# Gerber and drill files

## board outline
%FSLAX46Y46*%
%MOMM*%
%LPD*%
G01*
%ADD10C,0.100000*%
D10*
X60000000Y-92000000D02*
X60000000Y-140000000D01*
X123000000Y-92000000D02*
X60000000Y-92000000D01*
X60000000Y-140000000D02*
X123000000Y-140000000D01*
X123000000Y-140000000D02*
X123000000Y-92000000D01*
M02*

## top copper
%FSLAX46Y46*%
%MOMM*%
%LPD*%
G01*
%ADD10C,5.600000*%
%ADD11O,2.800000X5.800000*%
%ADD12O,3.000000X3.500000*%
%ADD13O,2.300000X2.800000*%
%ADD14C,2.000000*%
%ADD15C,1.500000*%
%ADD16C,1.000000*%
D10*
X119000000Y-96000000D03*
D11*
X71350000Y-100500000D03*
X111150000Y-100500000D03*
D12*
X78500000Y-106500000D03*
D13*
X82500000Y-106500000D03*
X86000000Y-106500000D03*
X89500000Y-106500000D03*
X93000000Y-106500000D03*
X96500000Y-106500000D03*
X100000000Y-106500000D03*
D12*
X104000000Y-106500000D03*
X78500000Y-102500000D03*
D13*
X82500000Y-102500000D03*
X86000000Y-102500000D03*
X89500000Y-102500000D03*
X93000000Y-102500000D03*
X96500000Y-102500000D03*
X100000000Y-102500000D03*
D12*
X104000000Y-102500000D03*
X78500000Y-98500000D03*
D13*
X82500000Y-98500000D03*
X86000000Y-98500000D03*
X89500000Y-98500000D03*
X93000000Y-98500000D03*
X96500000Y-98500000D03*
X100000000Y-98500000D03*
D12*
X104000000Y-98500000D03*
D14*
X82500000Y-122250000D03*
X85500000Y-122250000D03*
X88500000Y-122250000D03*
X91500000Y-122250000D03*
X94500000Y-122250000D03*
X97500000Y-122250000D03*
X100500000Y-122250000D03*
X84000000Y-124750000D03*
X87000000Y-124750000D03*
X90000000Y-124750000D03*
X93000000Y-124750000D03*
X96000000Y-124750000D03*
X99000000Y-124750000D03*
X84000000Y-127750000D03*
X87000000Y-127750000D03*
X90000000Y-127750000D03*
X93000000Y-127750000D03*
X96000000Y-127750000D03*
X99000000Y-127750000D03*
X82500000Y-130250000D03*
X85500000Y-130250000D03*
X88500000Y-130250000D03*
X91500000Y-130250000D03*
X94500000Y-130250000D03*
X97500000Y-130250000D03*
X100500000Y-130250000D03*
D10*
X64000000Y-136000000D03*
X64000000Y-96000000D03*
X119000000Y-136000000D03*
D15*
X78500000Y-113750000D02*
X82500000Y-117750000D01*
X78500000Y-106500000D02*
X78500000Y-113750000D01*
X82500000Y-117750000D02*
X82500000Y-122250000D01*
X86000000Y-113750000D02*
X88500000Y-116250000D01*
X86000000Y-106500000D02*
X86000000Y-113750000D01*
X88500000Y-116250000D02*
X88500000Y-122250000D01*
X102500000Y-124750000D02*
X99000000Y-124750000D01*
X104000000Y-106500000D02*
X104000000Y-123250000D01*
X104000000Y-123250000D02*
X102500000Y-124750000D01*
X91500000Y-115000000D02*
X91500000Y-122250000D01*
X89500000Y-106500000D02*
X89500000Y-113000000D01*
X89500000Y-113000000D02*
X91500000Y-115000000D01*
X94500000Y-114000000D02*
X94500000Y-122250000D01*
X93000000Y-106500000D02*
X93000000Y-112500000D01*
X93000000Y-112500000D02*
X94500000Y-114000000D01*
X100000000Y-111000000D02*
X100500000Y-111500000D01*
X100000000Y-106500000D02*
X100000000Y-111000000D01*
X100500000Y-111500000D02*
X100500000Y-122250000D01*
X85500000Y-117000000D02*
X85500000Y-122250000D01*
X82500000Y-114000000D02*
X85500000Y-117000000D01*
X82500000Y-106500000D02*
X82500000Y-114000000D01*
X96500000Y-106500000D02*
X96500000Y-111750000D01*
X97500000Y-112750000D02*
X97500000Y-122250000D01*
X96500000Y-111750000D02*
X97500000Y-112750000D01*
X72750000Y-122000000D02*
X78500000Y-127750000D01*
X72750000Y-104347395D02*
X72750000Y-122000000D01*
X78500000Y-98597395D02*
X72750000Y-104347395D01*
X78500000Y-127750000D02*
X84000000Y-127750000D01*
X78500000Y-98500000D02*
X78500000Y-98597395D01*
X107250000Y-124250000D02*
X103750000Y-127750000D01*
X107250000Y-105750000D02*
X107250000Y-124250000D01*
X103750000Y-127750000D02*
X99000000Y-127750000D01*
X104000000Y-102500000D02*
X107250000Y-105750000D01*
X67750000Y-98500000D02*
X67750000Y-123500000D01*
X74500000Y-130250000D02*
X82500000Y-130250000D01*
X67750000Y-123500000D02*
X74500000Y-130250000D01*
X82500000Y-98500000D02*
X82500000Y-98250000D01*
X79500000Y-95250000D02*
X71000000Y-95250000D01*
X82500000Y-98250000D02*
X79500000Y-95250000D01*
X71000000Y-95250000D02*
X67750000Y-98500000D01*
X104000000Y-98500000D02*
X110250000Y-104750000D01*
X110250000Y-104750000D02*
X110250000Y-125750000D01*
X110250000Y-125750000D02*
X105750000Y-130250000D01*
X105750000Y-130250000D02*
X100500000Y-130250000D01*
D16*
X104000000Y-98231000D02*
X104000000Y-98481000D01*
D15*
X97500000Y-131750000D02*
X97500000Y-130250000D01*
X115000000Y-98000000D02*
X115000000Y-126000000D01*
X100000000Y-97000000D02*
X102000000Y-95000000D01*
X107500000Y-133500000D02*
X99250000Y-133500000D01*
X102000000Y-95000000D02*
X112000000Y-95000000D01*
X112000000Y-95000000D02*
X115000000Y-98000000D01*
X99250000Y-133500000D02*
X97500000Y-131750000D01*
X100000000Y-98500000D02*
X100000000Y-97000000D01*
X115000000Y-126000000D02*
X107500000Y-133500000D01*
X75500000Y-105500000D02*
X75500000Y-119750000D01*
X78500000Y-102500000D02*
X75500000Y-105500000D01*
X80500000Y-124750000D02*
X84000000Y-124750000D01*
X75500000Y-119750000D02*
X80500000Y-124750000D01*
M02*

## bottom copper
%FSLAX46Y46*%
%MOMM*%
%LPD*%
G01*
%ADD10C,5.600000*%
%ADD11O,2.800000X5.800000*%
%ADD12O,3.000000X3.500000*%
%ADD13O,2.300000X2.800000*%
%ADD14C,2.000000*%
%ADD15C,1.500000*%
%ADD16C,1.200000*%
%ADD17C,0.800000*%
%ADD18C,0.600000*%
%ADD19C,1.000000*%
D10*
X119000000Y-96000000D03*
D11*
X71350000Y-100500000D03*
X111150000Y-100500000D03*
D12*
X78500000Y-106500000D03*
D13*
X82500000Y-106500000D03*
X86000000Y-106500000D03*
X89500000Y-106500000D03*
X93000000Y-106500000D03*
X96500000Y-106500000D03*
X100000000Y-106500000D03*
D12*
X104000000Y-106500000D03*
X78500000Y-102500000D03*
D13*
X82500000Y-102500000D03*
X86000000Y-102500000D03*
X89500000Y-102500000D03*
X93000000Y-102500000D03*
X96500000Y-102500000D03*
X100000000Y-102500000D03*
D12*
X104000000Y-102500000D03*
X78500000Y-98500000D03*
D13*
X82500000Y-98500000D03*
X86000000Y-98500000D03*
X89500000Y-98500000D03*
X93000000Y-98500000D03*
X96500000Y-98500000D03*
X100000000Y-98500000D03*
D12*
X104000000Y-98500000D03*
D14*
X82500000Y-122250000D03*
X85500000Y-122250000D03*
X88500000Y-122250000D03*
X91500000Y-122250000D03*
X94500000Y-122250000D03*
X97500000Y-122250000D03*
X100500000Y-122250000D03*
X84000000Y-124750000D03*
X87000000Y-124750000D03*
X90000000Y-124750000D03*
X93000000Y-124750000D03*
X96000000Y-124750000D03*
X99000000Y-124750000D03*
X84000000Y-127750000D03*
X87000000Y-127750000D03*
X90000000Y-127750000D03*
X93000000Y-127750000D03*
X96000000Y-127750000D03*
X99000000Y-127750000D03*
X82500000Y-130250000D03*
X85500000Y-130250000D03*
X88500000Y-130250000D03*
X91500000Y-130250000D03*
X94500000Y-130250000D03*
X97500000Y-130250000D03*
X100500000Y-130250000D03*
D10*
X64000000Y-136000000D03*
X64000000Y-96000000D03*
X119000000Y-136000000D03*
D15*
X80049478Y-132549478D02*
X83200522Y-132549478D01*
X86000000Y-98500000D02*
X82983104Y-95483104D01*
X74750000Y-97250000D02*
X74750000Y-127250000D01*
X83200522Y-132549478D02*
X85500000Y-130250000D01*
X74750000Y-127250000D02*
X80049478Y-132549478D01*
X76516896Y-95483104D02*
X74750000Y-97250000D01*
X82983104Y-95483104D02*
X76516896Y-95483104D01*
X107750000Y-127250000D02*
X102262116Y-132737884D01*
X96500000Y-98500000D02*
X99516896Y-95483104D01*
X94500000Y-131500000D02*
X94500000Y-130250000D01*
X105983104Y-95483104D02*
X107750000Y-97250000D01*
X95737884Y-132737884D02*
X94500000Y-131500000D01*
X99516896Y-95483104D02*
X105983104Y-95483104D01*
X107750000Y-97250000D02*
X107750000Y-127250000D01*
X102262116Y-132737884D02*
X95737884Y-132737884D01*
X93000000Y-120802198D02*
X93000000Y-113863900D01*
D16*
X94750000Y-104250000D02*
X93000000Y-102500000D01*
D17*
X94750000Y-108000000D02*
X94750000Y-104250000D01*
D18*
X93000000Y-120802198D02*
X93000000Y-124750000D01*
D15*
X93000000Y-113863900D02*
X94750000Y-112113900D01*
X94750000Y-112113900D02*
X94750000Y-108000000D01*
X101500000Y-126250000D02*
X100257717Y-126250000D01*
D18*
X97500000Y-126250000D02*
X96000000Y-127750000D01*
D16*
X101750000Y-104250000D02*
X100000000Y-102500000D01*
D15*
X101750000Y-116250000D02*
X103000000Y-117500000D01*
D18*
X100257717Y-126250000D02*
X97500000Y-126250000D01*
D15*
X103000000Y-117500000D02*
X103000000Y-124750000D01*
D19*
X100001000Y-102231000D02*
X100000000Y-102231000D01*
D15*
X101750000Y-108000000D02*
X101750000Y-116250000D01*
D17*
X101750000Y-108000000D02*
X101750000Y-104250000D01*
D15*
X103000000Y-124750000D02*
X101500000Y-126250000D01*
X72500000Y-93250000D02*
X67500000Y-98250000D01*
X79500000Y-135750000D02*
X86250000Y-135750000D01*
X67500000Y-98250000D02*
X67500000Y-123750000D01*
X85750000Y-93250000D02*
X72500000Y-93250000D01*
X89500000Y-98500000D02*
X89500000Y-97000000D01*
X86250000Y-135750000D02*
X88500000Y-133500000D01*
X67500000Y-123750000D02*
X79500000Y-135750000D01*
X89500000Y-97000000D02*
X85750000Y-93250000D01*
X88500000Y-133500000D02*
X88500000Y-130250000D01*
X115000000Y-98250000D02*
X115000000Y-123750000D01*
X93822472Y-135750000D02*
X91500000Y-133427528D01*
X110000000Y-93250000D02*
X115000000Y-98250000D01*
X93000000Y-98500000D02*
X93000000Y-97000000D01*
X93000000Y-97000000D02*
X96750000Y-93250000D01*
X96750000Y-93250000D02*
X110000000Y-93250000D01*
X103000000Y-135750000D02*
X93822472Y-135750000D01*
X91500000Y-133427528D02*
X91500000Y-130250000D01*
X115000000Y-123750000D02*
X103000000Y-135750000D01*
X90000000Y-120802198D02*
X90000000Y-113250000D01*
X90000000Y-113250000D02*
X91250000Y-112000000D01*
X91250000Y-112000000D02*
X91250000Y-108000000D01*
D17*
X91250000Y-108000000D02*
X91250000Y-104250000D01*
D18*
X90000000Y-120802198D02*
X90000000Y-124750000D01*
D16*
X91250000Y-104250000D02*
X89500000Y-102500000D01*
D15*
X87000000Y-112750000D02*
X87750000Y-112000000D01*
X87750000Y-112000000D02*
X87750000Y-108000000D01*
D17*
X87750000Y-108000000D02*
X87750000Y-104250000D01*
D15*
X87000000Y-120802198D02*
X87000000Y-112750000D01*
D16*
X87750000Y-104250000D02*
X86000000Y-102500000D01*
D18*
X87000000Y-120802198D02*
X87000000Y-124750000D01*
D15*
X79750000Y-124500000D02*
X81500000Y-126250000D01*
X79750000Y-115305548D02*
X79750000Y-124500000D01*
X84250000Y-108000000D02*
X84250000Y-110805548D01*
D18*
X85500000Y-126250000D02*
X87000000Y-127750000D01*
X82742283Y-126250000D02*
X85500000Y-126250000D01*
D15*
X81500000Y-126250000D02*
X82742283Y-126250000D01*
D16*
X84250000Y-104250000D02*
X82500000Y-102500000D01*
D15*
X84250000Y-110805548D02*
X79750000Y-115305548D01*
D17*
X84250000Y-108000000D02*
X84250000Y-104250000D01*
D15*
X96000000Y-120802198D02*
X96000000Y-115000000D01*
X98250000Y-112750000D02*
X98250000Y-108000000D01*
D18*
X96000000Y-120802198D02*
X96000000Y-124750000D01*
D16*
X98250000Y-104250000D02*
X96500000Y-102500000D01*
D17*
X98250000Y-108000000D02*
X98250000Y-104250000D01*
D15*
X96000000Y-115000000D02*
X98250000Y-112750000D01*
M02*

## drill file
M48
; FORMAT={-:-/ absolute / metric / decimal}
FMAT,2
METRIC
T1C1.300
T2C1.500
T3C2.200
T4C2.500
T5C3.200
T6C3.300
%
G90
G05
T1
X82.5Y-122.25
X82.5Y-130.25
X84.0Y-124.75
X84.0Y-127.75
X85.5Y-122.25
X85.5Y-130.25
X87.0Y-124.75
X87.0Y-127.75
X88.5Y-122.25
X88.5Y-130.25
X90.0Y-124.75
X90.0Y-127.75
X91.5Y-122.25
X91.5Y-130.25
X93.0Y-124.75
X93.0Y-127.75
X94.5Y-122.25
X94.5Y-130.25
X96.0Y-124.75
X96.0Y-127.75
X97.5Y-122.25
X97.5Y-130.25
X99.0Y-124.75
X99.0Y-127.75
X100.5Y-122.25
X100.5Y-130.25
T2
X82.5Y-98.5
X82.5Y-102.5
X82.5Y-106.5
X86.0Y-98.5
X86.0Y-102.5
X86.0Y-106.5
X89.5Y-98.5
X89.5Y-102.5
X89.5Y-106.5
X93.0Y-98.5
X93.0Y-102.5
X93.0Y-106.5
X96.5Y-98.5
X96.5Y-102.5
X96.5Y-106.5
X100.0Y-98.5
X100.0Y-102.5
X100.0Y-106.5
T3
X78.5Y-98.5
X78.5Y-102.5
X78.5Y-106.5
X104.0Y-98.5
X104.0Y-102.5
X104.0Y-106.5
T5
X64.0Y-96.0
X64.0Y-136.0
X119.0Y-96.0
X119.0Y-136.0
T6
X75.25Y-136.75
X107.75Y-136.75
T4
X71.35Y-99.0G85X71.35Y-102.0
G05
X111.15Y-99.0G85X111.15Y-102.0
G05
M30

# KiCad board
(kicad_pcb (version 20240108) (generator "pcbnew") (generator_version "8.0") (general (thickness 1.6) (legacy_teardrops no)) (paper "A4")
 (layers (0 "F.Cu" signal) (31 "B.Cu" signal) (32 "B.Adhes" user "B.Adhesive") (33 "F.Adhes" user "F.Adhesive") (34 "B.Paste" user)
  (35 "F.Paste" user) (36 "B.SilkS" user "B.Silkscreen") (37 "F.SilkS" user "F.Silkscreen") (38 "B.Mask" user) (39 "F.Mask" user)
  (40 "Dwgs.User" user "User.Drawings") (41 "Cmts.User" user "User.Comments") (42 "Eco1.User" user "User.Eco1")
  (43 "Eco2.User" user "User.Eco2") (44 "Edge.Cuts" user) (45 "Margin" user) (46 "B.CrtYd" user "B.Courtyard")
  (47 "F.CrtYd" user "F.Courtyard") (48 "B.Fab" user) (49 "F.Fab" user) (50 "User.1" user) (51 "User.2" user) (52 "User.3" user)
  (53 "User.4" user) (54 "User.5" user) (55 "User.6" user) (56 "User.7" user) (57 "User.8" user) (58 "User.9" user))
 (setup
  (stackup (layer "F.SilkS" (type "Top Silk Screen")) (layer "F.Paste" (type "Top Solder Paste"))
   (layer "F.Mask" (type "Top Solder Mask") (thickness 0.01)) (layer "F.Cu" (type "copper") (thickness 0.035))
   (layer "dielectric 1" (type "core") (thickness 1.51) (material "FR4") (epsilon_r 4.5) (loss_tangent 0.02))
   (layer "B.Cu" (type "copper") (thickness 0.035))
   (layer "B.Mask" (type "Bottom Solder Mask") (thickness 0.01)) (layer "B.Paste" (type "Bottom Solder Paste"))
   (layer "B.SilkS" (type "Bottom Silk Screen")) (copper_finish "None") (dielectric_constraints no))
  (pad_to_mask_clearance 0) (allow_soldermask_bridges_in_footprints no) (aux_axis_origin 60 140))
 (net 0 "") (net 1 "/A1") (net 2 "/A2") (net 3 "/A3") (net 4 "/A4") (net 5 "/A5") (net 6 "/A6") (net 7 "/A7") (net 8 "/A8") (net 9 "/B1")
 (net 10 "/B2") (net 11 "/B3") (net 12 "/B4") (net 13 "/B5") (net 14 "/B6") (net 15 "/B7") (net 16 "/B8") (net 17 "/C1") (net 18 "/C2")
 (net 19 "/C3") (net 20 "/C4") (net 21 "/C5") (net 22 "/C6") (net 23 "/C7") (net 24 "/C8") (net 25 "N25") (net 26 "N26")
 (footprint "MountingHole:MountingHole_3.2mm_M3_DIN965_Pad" (layer "F.Cu") (at 119 96 180)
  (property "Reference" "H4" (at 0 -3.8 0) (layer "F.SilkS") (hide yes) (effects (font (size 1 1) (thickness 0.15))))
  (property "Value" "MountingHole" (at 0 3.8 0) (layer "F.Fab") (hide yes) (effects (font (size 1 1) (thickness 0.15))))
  (pad "1" thru_hole circle (at 0 0 180) (size 5.6 5.6) (drill 3.2) (layers "*.Cu" "*.Mask") (remove_unused_layers no)))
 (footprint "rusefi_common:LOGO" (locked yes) (layer "F.Cu") (at 67.36 115.1)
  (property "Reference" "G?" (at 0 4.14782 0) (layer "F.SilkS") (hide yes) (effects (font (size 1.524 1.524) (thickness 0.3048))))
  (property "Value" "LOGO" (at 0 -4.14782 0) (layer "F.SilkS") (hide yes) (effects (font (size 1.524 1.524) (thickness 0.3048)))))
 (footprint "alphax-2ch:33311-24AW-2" (layer "F.Cu") (at 78.5 106.5)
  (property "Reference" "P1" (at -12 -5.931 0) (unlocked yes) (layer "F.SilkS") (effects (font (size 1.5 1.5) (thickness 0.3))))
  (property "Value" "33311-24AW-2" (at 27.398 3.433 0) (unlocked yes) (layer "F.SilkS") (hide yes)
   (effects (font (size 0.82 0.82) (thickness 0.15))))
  (pad "" thru_hole oval (at -7.15 -6 270) (size 5.8 2.8) (drill oval 5.5 2.5) (layers "*.Cu" "*.Mask") (remove_unused_layers no)
   (solder_mask_margin 0.05))
  (pad "" thru_hole oval (at 32.65 -6 270) (size 5.8 2.8) (drill oval 5.5 2.5) (layers "*.Cu" "*.Mask") (remove_unused_layers no)
   (solder_mask_margin 0.05))
  (pad "1" thru_hole oval (at 0 0 270) (size 3.5 3) (drill 2.2) (layers "*.Cu" "*.Mask") (remove_unused_layers no) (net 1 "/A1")
   (solder_mask_margin 0.05))
  (pad "2" thru_hole oval (at 4 0 270) (size 2.8 2.3) (drill 1.5) (layers "*.Cu" "*.Mask") (remove_unused_layers no) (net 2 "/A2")
   (solder_mask_margin 0.05))
  (pad "3" thru_hole oval (at 7.5 0 270) (size 2.8 2.3) (drill 1.5) (layers "*.Cu" "*.Mask") (remove_unused_layers no) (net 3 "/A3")
   (solder_mask_margin 0.05))
  (pad "4" thru_hole oval (at 11 0 270) (size 2.8 2.3) (drill 1.5) (layers "*.Cu" "*.Mask") (remove_unused_layers no) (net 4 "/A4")
   (solder_mask_margin 0.05))
  (pad "5" thru_hole oval (at 14.5 0 270) (size 2.8 2.3) (drill 1.5) (layers "*.Cu" "*.Mask") (remove_unused_layers no) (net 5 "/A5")
   (solder_mask_margin 0.05))
  (pad "6" thru_hole oval (at 18 0 270) (size 2.8 2.3) (drill 1.5) (layers "*.Cu" "*.Mask") (remove_unused_layers no) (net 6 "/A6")
   (solder_mask_margin 0.05))
  (pad "7" thru_hole oval (at 21.5 0 270) (size 2.8 2.3) (drill 1.5) (layers "*.Cu" "*.Mask") (remove_unused_layers no) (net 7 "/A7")
   (solder_mask_margin 0.05))
  (pad "8" thru_hole oval (at 25.5 0 270) (size 3.5 3) (drill 2.2) (layers "*.Cu" "*.Mask") (remove_unused_layers no) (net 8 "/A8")
   (solder_mask_margin 0.05))
  (pad "9" thru_hole oval (at 0 -4 270) (size 3.5 3) (drill 2.2) (layers "*.Cu" "*.Mask") (remove_unused_layers no) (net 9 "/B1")
   (solder_mask_margin 0.05))
  (pad "10" thru_hole oval (at 4 -4 270) (size 2.8 2.3) (drill 1.5) (layers "*.Cu" "*.Mask") (remove_unused_layers no) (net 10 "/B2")
   (solder_mask_margin 0.05))
  (pad "11" thru_hole oval (at 7.5 -4 270) (size 2.8 2.3) (drill 1.5) (layers "*.Cu" "*.Mask") (remove_unused_layers no) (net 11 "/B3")
   (solder_mask_margin 0.05))
  (pad "12" thru_hole oval (at 11 -4 270) (size 2.8 2.3) (drill 1.5) (layers "*.Cu" "*.Mask") (remove_unused_layers no) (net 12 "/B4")
   (solder_mask_margin 0.05))
  (pad "13" thru_hole oval (at 14.5 -4 270) (size 2.8 2.3) (drill 1.5) (layers "*.Cu" "*.Mask") (remove_unused_layers no) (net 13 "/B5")
   (solder_mask_margin 0.05))
  (pad "14" thru_hole oval (at 18 -4 270) (size 2.8 2.3) (drill 1.5) (layers "*.Cu" "*.Mask") (remove_unused_layers no) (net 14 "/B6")
   (solder_mask_margin 0.05))
  (pad "15" thru_hole oval (at 21.5 -4 270) (size 2.8 2.3) (drill 1.5) (layers "*.Cu" "*.Mask") (remove_unused_layers no) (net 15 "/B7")
   (solder_mask_margin 0.05))
  (pad "16" thru_hole oval (at 25.5 -4 270) (size 3.5 3) (drill 2.2) (layers "*.Cu" "*.Mask") (remove_unused_layers no) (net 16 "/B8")
   (solder_mask_margin 0.05))
  (pad "17" thru_hole oval (at 0 -8 270) (size 3.5 3) (drill 2.2) (layers "*.Cu" "*.Mask") (remove_unused_layers no) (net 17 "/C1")
   (solder_mask_margin 0.05))
  (pad "18" thru_hole oval (at 4 -8 270) (size 2.8 2.3) (drill 1.5) (layers "*.Cu" "*.Mask") (remove_unused_layers no) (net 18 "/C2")
   (solder_mask_margin 0.05))
  (pad "19" thru_hole oval (at 7.5 -8 270) (size 2.8 2.3) (drill 1.5) (layers "*.Cu" "*.Mask") (remove_unused_layers no) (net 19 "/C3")
   (solder_mask_margin 0.05))
  (pad "20" thru_hole oval (at 11 -8 270) (size 2.8 2.3) (drill 1.5) (layers "*.Cu" "*.Mask") (remove_unused_layers no) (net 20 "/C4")
   (solder_mask_margin 0.05))
  (pad "21" thru_hole oval (at 14.5 -8 270) (size 2.8 2.3) (drill 1.5) (layers "*.Cu" "*.Mask") (remove_unused_layers no) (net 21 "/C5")
   (solder_mask_margin 0.05))
  (pad "22" thru_hole oval (at 18 -8 270) (size 2.8 2.3) (drill 1.5) (layers "*.Cu" "*.Mask") (remove_unused_layers no) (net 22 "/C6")
   (solder_mask_margin 0.05))
  (pad "23" thru_hole oval (at 21.5 -8 270) (size 2.8 2.3) (drill 1.5) (layers "*.Cu" "*.Mask") (remove_unused_layers no) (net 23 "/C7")
   (solder_mask_margin 0.05))
  (pad "24" thru_hole oval (at 25.5 -8 270) (size 3.5 3) (drill 2.2) (layers "*.Cu" "*.Mask") (remove_unused_layers no) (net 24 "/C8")
   (solder_mask_margin 0.05)))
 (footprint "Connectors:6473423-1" (layer "F.Cu") (at 91.5 136.75)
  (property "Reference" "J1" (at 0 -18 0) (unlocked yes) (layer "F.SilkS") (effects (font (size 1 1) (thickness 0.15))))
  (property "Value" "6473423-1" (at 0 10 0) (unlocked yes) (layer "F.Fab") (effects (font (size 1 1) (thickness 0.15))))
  (pad "" np_thru_hole circle (at -16.25 0) (size 3.3 3.3) (drill 3.3) (layers "F&B.Cu" "*.Mask"))
  (pad "" np_thru_hole circle (at 16.25 0) (size 3.3 3.3) (drill 3.3) (layers "F&B.Cu" "*.Mask"))
  (pad "1" thru_hole circle (at -9 -14.5 270) (size 2 2) (drill 1.3) (layers "*.Cu" "*.Mask") (remove_unused_layers no) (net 1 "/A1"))
  (pad "2" thru_hole circle (at -6 -14.5) (size 2 2) (drill 1.3) (layers "*.Cu" "*.Mask") (remove_unused_layers no) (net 2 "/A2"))
  (pad "3" thru_hole circle (at -3 -14.5) (size 2 2) (drill 1.3) (layers "*.Cu" "*.Mask") (remove_unused_layers no) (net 3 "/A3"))
  (pad "4" thru_hole circle (at 0 -14.5) (size 2 2) (drill 1.3) (layers "*.Cu" "*.Mask") (remove_unused_layers no) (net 4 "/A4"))
  (pad "5" thru_hole circle (at 3 -14.5 270) (size 2 2) (drill 1.3) (layers "*.Cu" "*.Mask") (remove_unused_layers no) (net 5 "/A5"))
  (pad "6" thru_hole circle (at 6 -14.5) (size 2 2) (drill 1.3) (layers "*.Cu" "*.Mask") (remove_unused_layers no) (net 6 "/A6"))
  (pad "7" thru_hole circle (at 9 -14.5) (size 2 2) (drill 1.3) (layers "*.Cu" "*.Mask") (remove_unused_layers no) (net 7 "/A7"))
  (pad "8" thru_hole circle (at -7.5 -12 270) (size 2 2) (drill 1.3) (layers "*.Cu" "*.Mask") (remove_unused_layers no) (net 9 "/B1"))
  (pad "9" thru_hole circle (at -4.5 -12) (size 2 2) (drill 1.3) (layers "*.Cu" "*.Mask") (remove_unused_layers no) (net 11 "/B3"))
  (pad "10" thru_hole circle (at -1.5 -12) (size 2 2) (drill 1.3) (layers "*.Cu" "*.Mask") (remove_unused_layers no) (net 12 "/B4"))
  (pad "11" thru_hole circle (at 1.5 -12) (size 2 2) (drill 1.3) (layers "*.Cu" "*.Mask") (remove_unused_layers no) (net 13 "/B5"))
  (pad "12" thru_hole circle (at 4.5 -12 270) (size 2 2) (drill 1.3) (layers "*.Cu" "*.Mask") (remove_unused_layers no) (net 14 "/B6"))
  (pad "13" thru_hole circle (at 7.5 -12) (size 2 2) (drill 1.3) (layers "*.Cu" "*.Mask") (remove_unused_layers no) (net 8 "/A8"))
  (pad "14" thru_hole circle (at -7.5 -9 270) (size 2 2) (drill 1.3) (layers "*.Cu" "*.Mask") (remove_unused_layers no) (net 17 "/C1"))
  (pad "15" thru_hole circle (at -4.5 -9) (size 2 2) (drill 1.3) (layers "*.Cu" "*.Mask") (remove_unused_layers no) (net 10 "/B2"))
  (pad "16" thru_hole circle (at -1.5 -9) (size 2 2) (drill 1.3) (layers "*.Cu" "*.Mask") (remove_unused_layers no) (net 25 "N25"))
  (pad "17" thru_hole circle (at 1.5 -9) (size 2 2) (drill 1.3) (layers "*.Cu" "*.Mask") (remove_unused_layers no) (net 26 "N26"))
  (pad "18" thru_hole circle (at 4.5 -9 270) (size 2 2) (drill 1.3) (layers "*.Cu" "*.Mask") (remove_unused_layers no) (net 15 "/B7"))
  (pad "19" thru_hole circle (at 7.5 -9) (size 2 2) (drill 1.3) (layers "*.Cu" "*.Mask") (remove_unused_layers no) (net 16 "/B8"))
  (pad "20" thru_hole circle (at -9 -6.5 270) (size 2 2) (drill 1.3) (layers "*.Cu" "*.Mask") (remove_unused_layers no) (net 18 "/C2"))
  (pad "21" thru_hole circle (at -6 -6.5) (size 2 2) (drill 1.3) (layers "*.Cu" "*.Mask") (remove_unused_layers no) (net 19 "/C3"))
  (pad "22" thru_hole circle (at -3 -6.5) (size 2 2) (drill 1.3) (layers "*.Cu" "*.Mask") (remove_unused_layers no) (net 20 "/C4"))
  (pad "23" thru_hole circle (at 0 -6.5) (size 2 2) (drill 1.3) (layers "*.Cu" "*.Mask") (remove_unused_layers no) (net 21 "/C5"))
  (pad "24" thru_hole circle (at 3 -6.5 270) (size 2 2) (drill 1.3) (layers "*.Cu" "*.Mask") (remove_unused_layers no) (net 22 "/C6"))
  (pad "25" thru_hole circle (at 6 -6.5) (size 2 2) (drill 1.3) (layers "*.Cu" "*.Mask") (remove_unused_layers no) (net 23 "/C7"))
  (pad "26" thru_hole circle (at 9 -6.5) (size 2 2) (drill 1.3) (layers "*.Cu" "*.Mask") (remove_unused_layers no) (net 24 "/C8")))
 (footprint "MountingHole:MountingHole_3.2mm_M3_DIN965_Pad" (layer "F.Cu") (at 64 136 180)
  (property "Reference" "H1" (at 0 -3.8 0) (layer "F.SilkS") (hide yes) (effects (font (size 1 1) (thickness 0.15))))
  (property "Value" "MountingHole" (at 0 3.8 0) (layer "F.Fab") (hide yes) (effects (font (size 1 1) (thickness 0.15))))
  (pad "1" thru_hole circle (at 0 0 180) (size 5.6 5.6) (drill 3.2) (layers "*.Cu" "*.Mask") (remove_unused_layers no)))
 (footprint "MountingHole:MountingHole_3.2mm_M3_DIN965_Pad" (layer "F.Cu") (at 64 96 180)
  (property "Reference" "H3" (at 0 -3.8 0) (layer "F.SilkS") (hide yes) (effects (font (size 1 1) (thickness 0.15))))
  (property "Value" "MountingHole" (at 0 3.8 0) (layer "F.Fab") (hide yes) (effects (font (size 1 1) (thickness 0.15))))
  (pad "1" thru_hole circle (at 0 0 180) (size 5.6 5.6) (drill 3.2) (layers "*.Cu" "*.Mask") (remove_unused_layers no)))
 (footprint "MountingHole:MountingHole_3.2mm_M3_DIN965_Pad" (layer "F.Cu") (at 119 136 180)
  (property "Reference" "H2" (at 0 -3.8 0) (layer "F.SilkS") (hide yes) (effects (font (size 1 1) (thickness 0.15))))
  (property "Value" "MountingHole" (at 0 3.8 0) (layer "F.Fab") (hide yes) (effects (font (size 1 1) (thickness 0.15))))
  (pad "1" thru_hole circle (at 0 0 180) (size 5.6 5.6) (drill 3.2) (layers "*.Cu" "*.Mask") (remove_unused_layers no)))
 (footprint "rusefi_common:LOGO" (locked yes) (layer "B.Cu") (at 114.934286 115.2 180)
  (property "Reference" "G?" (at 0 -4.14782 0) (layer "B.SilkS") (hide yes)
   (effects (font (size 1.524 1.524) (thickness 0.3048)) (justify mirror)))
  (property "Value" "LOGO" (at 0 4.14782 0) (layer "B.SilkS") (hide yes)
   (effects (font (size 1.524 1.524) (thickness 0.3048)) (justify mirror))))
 (gr_line (start 60 92) (end 60 140) (stroke (width 0.1) (type solid)) (layer "Edge.Cuts"))
 (gr_line (start 123 92) (end 60 92) (stroke (width 0.1) (type solid)) (layer "Edge.Cuts"))
 (gr_line (start 60 140) (end 123 140) (stroke (width 0.1) (type solid)) (layer "Edge.Cuts"))
 (gr_line (start 123 140) (end 123 92) (stroke (width 0.1) (type solid)) (layer "Edge.Cuts"))
 (segment (start 78.5 113.75) (end 82.5 117.75) (width 1.5) (layer "F.Cu") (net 1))
 (segment (start 78.5 106.5) (end 78.5 113.75) (width 1.5) (layer "F.Cu") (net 1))
 (segment (start 82.5 117.75) (end 82.5 122.25) (width 1.5) (layer "F.Cu") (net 1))
 (segment (start 86 113.75) (end 88.5 116.25) (width 1.5) (layer "F.Cu") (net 3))
 (segment (start 86 106.5) (end 86 113.75) (width 1.5) (layer "F.Cu") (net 3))
 (segment (start 88.5 116.25) (end 88.5 122.25) (width 1.5) (layer "F.Cu") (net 3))
 (segment (start 102.5 124.75) (end 99 124.75) (width 1.5) (layer "F.Cu") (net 8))
 (segment (start 104 106.5) (end 104 123.25) (width 1.5) (layer "F.Cu") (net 8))
 (segment (start 104 123.25) (end 102.5 124.75) (width 1.5) (layer "F.Cu") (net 8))
 (segment (start 91.5 115) (end 91.5 122.25) (width 1.5) (layer "F.Cu") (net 4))
 (segment (start 89.5 106.5) (end 89.5 113) (width 1.5) (layer "F.Cu") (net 4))
 (segment (start 89.5 113) (end 91.5 115) (width 1.5) (layer "F.Cu") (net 4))
 (segment (start 94.5 114) (end 94.5 122.25) (width 1.5) (layer "F.Cu") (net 5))
 (segment (start 93 106.5) (end 93 112.5) (width 1.5) (layer "F.Cu") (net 5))
 (segment (start 93 112.5) (end 94.5 114) (width 1.5) (layer "F.Cu") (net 5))
 (segment (start 100 111) (end 100.5 111.5) (width 1.5) (layer "F.Cu") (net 7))
 (segment (start 100 106.5) (end 100 111) (width 1.5) (layer "F.Cu") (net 7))
 (segment (start 100.5 111.5) (end 100.5 122.25) (width 1.5) (layer "F.Cu") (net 7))
 (segment (start 85.5 117) (end 85.5 122.25) (width 1.5) (layer "F.Cu") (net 2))
 (segment (start 82.5 114) (end 85.5 117) (width 1.5) (layer "F.Cu") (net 2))
 (segment (start 82.5 106.5) (end 82.5 114) (width 1.5) (layer "F.Cu") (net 2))
 (segment (start 96.5 106.5) (end 96.5 111.75) (width 1.5) (layer "F.Cu") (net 6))
 (segment (start 97.5 112.75) (end 97.5 122.25) (width 1.5) (layer "F.Cu") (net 6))
 (segment (start 96.5 111.75) (end 97.5 112.75) (width 1.5) (layer "F.Cu") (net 6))
 (segment (start 80.049478 132.549478) (end 83.200522 132.549478) (width 1.5) (layer "B.Cu") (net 19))
 (segment (start 86 98.5) (end 82.983104 95.483104) (width 1.5) (layer "B.Cu") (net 19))
 (segment (start 74.75 97.25) (end 74.75 127.25) (width 1.5) (layer "B.Cu") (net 19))
 (segment (start 83.200522 132.549478) (end 85.5 130.25) (width 1.5) (layer "B.Cu") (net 19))
 (segment (start 74.75 127.25) (end 80.049478 132.549478) (width 1.5) (layer "B.Cu") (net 19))
 (segment (start 76.516896 95.483104) (end 74.75 97.25) (width 1.5) (layer "B.Cu") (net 19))
 (segment (start 82.983104 95.483104) (end 76.516896 95.483104) (width 1.5) (layer "B.Cu") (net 19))
 (segment (start 107.75 127.25) (end 102.262116 132.737884) (width 1.5) (layer "B.Cu") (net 22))
 (segment (start 96.5 98.5) (end 99.516896 95.483104) (width 1.5) (layer "B.Cu") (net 22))
 (segment (start 94.5 131.5) (end 94.5 130.25) (width 1.5) (layer "B.Cu") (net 22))
 (segment (start 105.983104 95.483104) (end 107.75 97.25) (width 1.5) (layer "B.Cu") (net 22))
 (segment (start 95.737884 132.737884) (end 94.5 131.5) (width 1.5) (layer "B.Cu") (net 22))
 (segment (start 99.516896 95.483104) (end 105.983104 95.483104) (width 1.5) (layer "B.Cu") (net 22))
 (segment (start 107.75 97.25) (end 107.75 127.25) (width 1.5) (layer "B.Cu") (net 22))
 (segment (start 102.262116 132.737884) (end 95.737884 132.737884) (width 1.5) (layer "B.Cu") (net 22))
 (segment (start 72.75 122) (end 78.5 127.75) (width 1.5) (layer "F.Cu") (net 17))
 (segment (start 72.75 104.347395) (end 72.75 122) (width 1.5) (layer "F.Cu") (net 17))
 (segment (start 78.5 98.597395) (end 72.75 104.347395) (width 1.5) (layer "F.Cu") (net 17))
 (segment (start 78.5 127.75) (end 84 127.75) (width 1.5) (layer "F.Cu") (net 17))
 (segment (start 78.5 98.5) (end 78.5 98.597395) (width 1.5) (layer "F.Cu") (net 17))
 (segment (start 107.25 124.25) (end 103.75 127.75) (width 1.5) (layer "F.Cu") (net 16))
 (segment (start 107.25 105.75) (end 107.25 124.25) (width 1.5) (layer "F.Cu") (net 16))
 (segment (start 103.75 127.75) (end 99 127.75) (width 1.5) (layer "F.Cu") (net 16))
 (segment (start 104 102.5) (end 107.25 105.75) (width 1.5) (layer "F.Cu") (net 16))
 (segment (start 93 120.802198) (end 93 113.8639) (width 1.5) (layer "B.Cu") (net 13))
 (segment (start 94.75 104.25) (end 93 102.5) (width 1.2) (layer "B.Cu") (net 13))
 (segment (start 94.75 108) (end 94.75 104.25) (width 0.8) (layer "B.Cu") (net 13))
 (segment (start 93 120.802198) (end 93 124.75) (width 0.6) (layer "B.Cu") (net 13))
 (segment (start 93 113.8639) (end 94.75 112.1139) (width 1.5) (layer "B.Cu") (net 13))
 (segment (start 94.75 112.1139) (end 94.75 108) (width 1.5) (layer "B.Cu") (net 13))
 (segment (start 101.5 126.25) (end 100.257717 126.25) (width 1.5) (layer "B.Cu") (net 15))
 (segment (start 97.5 126.25) (end 96 127.75) (width 0.6) (layer "B.Cu") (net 15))
 (segment (start 101.75 104.25) (end 100 102.5) (width 1.2) (layer "B.Cu") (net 15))
 (segment (start 101.75 116.25) (end 103 117.5) (width 1.5) (layer "B.Cu") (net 15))
 (segment (start 100.257717 126.25) (end 97.5 126.25) (width 0.6) (layer "B.Cu") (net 15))
 (segment (start 103 117.5) (end 103 124.75) (width 1.5) (layer "B.Cu") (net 15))
 (segment (start 100.001 102.231) (end 100 102.231) (width 1) (layer "B.Cu") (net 15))
 (segment (start 101.75 108) (end 101.75 116.25) (width 1.5) (layer "B.Cu") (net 15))
 (segment (start 101.75 108) (end 101.75 104.25) (width 0.8) (layer "B.Cu") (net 15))
 (segment (start 103 124.75) (end 101.5 126.25) (width 1.5) (layer "B.Cu") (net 15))
 (segment (start 67.75 98.5) (end 67.75 123.5) (width 1.5) (layer "F.Cu") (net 18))
 (segment (start 74.5 130.25) (end 82.5 130.25) (width 1.5) (layer "F.Cu") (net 18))
 (segment (start 67.75 123.5) (end 74.5 130.25) (width 1.5) (layer "F.Cu") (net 18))
 (segment (start 82.5 98.5) (end 82.5 98.25) (width 1.5) (layer "F.Cu") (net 18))
 (segment (start 79.5 95.25) (end 71 95.25) (width 1.5) (layer "F.Cu") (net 18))
 (segment (start 82.5 98.25) (end 79.5 95.25) (width 1.5) (layer "F.Cu") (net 18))
 (segment (start 71 95.25) (end 67.75 98.5) (width 1.5) (layer "F.Cu") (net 18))
 (segment (start 72.5 93.25) (end 67.5 98.25) (width 1.5) (layer "B.Cu") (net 20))
 (segment (start 79.5 135.75) (end 86.25 135.75) (width 1.5) (layer "B.Cu") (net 20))
 (segment (start 67.5 98.25) (end 67.5 123.75) (width 1.5) (layer "B.Cu") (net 20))
 (segment (start 85.75 93.25) (end 72.5 93.25) (width 1.5) (layer "B.Cu") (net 20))
 (segment (start 89.5 98.5) (end 89.5 97) (width 1.5) (layer "B.Cu") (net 20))
 (segment (start 86.25 135.75) (end 88.5 133.5) (width 1.5) (layer "B.Cu") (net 20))
 (segment (start 67.5 123.75) (end 79.5 135.75) (width 1.5) (layer "B.Cu") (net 20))
 (segment (start 89.5 97) (end 85.75 93.25) (width 1.5) (layer "B.Cu") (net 20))
 (segment (start 88.5 133.5) (end 88.5 130.25) (width 1.5) (layer "B.Cu") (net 20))
 (segment (start 104 98.5) (end 110.25 104.75) (width 1.5) (layer "F.Cu") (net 24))
 (segment (start 110.25 104.75) (end 110.25 125.75) (width 1.5) (layer "F.Cu") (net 24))
 (segment (start 110.25 125.75) (end 105.75 130.25) (width 1.5) (layer "F.Cu") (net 24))
 (segment (start 105.75 130.25) (end 100.5 130.25) (width 1.5) (layer "F.Cu") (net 24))
 (segment (start 104 98.231) (end 104 98.481) (width 1) (layer "F.Cu") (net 24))
 (segment (start 115 98.25) (end 115 123.75) (width 1.5) (layer "B.Cu") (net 21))
 (segment (start 93.822472 135.75) (end 91.5 133.427528) (width 1.5) (layer "B.Cu") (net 21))
 (segment (start 110 93.25) (end 115 98.25) (width 1.5) (layer "B.Cu") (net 21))
 (segment (start 93 98.5) (end 93 97) (width 1.5) (layer "B.Cu") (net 21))
 (segment (start 93 97) (end 96.75 93.25) (width 1.5) (layer "B.Cu") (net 21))
 (segment (start 96.75 93.25) (end 110 93.25) (width 1.5) (layer "B.Cu") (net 21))
 (segment (start 103 135.75) (end 93.822472 135.75) (width 1.5) (layer "B.Cu") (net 21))
 (segment (start 91.5 133.427528) (end 91.5 130.25) (width 1.5) (layer "B.Cu") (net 21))
 (segment (start 115 123.75) (end 103 135.75) (width 1.5) (layer "B.Cu") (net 21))
 (segment (start 90 120.802198) (end 90 113.25) (width 1.5) (layer "B.Cu") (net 12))
 (segment (start 90 113.25) (end 91.25 112) (width 1.5) (layer "B.Cu") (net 12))
 (segment (start 91.25 112) (end 91.25 108) (width 1.5) (layer "B.Cu") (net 12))
 (segment (start 91.25 108) (end 91.25 104.25) (width 0.8) (layer "B.Cu") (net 12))
 (segment (start 90 120.802198) (end 90 124.75) (width 0.6) (layer "B.Cu") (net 12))
 (segment (start 91.25 104.25) (end 89.5 102.5) (width 1.2) (layer "B.Cu") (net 12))
 (segment (start 97.5 131.75) (end 97.5 130.25) (width 1.5) (layer "F.Cu") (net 23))
 (segment (start 115 98) (end 115 126) (width 1.5) (layer "F.Cu") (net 23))
 (segment (start 100 97) (end 102 95) (width 1.5) (layer "F.Cu") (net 23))
 (segment (start 107.5 133.5) (end 99.25 133.5) (width 1.5) (layer "F.Cu") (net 23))
 (segment (start 102 95) (end 112 95) (width 1.5) (layer "F.Cu") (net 23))
 (segment (start 112 95) (end 115 98) (width 1.5) (layer "F.Cu") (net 23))
 (segment (start 99.25 133.5) (end 97.5 131.75) (width 1.5) (layer "F.Cu") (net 23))
 (segment (start 100 98.5) (end 100 97) (width 1.5) (layer "F.Cu") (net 23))
 (segment (start 115 126) (end 107.5 133.5) (width 1.5) (layer "F.Cu") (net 23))
 (segment (start 75.5 105.5) (end 75.5 119.75) (width 1.5) (layer "F.Cu") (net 9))
 (segment (start 78.5 102.5) (end 75.5 105.5) (width 1.5) (layer "F.Cu") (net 9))
 (segment (start 80.5 124.75) (end 84 124.75) (width 1.5) (layer "F.Cu") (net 9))
 (segment (start 75.5 119.75) (end 80.5 124.75) (width 1.5) (layer "F.Cu") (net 9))
 (segment (start 87 112.75) (end 87.75 112) (width 1.5) (layer "B.Cu") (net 11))
 (segment (start 87.75 112) (end 87.75 108) (width 1.5) (layer "B.Cu") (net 11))
 (segment (start 87.75 108) (end 87.75 104.25) (width 0.8) (layer "B.Cu") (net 11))
 (segment (start 87 120.802198) (end 87 112.75) (width 1.5) (layer "B.Cu") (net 11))
 (segment (start 87.75 104.25) (end 86 102.5) (width 1.2) (layer "B.Cu") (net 11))
 (segment (start 87 120.802198) (end 87 124.75) (width 0.6) (layer "B.Cu") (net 11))
 (segment (start 79.75 124.5) (end 81.5 126.25) (width 1.5) (layer "B.Cu") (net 10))
 (segment (start 79.75 115.305548) (end 79.75 124.5) (width 1.5) (layer "B.Cu") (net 10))
 (segment (start 84.25 108) (end 84.25 110.805548) (width 1.5) (layer "B.Cu") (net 10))
 (segment (start 85.5 126.25) (end 87 127.75) (width 0.6) (layer "B.Cu") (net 10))
 (segment (start 82.742283 126.25) (end 85.5 126.25) (width 0.6) (layer "B.Cu") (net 10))
 (segment (start 81.5 126.25) (end 82.742283 126.25) (width 1.5) (layer "B.Cu") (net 10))
 (segment (start 84.25 104.25) (end 82.5 102.5) (width 1.2) (layer "B.Cu") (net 10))
 (segment (start 84.25 110.805548) (end 79.75 115.305548) (width 1.5) (layer "B.Cu") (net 10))
 (segment (start 84.25 108) (end 84.25 104.25) (width 0.8) (layer "B.Cu") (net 10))
 (segment (start 96 120.802198) (end 96 115) (width 1.5) (layer "B.Cu") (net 14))
 (segment (start 98.25 112.75) (end 98.25 108) (width 1.5) (layer "B.Cu") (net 14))
 (segment (start 96 120.802198) (end 96 124.75) (width 0.6) (layer "B.Cu") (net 14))
 (segment (start 98.25 104.25) (end 96.5 102.5) (width 1.2) (layer "B.Cu") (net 14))
 (segment (start 98.25 108) (end 98.25 104.25) (width 0.8) (layer "B.Cu") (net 14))
 (segment (start 96 115) (end 98.25 112.75) (width 1.5) (layer "B.Cu") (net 14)))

